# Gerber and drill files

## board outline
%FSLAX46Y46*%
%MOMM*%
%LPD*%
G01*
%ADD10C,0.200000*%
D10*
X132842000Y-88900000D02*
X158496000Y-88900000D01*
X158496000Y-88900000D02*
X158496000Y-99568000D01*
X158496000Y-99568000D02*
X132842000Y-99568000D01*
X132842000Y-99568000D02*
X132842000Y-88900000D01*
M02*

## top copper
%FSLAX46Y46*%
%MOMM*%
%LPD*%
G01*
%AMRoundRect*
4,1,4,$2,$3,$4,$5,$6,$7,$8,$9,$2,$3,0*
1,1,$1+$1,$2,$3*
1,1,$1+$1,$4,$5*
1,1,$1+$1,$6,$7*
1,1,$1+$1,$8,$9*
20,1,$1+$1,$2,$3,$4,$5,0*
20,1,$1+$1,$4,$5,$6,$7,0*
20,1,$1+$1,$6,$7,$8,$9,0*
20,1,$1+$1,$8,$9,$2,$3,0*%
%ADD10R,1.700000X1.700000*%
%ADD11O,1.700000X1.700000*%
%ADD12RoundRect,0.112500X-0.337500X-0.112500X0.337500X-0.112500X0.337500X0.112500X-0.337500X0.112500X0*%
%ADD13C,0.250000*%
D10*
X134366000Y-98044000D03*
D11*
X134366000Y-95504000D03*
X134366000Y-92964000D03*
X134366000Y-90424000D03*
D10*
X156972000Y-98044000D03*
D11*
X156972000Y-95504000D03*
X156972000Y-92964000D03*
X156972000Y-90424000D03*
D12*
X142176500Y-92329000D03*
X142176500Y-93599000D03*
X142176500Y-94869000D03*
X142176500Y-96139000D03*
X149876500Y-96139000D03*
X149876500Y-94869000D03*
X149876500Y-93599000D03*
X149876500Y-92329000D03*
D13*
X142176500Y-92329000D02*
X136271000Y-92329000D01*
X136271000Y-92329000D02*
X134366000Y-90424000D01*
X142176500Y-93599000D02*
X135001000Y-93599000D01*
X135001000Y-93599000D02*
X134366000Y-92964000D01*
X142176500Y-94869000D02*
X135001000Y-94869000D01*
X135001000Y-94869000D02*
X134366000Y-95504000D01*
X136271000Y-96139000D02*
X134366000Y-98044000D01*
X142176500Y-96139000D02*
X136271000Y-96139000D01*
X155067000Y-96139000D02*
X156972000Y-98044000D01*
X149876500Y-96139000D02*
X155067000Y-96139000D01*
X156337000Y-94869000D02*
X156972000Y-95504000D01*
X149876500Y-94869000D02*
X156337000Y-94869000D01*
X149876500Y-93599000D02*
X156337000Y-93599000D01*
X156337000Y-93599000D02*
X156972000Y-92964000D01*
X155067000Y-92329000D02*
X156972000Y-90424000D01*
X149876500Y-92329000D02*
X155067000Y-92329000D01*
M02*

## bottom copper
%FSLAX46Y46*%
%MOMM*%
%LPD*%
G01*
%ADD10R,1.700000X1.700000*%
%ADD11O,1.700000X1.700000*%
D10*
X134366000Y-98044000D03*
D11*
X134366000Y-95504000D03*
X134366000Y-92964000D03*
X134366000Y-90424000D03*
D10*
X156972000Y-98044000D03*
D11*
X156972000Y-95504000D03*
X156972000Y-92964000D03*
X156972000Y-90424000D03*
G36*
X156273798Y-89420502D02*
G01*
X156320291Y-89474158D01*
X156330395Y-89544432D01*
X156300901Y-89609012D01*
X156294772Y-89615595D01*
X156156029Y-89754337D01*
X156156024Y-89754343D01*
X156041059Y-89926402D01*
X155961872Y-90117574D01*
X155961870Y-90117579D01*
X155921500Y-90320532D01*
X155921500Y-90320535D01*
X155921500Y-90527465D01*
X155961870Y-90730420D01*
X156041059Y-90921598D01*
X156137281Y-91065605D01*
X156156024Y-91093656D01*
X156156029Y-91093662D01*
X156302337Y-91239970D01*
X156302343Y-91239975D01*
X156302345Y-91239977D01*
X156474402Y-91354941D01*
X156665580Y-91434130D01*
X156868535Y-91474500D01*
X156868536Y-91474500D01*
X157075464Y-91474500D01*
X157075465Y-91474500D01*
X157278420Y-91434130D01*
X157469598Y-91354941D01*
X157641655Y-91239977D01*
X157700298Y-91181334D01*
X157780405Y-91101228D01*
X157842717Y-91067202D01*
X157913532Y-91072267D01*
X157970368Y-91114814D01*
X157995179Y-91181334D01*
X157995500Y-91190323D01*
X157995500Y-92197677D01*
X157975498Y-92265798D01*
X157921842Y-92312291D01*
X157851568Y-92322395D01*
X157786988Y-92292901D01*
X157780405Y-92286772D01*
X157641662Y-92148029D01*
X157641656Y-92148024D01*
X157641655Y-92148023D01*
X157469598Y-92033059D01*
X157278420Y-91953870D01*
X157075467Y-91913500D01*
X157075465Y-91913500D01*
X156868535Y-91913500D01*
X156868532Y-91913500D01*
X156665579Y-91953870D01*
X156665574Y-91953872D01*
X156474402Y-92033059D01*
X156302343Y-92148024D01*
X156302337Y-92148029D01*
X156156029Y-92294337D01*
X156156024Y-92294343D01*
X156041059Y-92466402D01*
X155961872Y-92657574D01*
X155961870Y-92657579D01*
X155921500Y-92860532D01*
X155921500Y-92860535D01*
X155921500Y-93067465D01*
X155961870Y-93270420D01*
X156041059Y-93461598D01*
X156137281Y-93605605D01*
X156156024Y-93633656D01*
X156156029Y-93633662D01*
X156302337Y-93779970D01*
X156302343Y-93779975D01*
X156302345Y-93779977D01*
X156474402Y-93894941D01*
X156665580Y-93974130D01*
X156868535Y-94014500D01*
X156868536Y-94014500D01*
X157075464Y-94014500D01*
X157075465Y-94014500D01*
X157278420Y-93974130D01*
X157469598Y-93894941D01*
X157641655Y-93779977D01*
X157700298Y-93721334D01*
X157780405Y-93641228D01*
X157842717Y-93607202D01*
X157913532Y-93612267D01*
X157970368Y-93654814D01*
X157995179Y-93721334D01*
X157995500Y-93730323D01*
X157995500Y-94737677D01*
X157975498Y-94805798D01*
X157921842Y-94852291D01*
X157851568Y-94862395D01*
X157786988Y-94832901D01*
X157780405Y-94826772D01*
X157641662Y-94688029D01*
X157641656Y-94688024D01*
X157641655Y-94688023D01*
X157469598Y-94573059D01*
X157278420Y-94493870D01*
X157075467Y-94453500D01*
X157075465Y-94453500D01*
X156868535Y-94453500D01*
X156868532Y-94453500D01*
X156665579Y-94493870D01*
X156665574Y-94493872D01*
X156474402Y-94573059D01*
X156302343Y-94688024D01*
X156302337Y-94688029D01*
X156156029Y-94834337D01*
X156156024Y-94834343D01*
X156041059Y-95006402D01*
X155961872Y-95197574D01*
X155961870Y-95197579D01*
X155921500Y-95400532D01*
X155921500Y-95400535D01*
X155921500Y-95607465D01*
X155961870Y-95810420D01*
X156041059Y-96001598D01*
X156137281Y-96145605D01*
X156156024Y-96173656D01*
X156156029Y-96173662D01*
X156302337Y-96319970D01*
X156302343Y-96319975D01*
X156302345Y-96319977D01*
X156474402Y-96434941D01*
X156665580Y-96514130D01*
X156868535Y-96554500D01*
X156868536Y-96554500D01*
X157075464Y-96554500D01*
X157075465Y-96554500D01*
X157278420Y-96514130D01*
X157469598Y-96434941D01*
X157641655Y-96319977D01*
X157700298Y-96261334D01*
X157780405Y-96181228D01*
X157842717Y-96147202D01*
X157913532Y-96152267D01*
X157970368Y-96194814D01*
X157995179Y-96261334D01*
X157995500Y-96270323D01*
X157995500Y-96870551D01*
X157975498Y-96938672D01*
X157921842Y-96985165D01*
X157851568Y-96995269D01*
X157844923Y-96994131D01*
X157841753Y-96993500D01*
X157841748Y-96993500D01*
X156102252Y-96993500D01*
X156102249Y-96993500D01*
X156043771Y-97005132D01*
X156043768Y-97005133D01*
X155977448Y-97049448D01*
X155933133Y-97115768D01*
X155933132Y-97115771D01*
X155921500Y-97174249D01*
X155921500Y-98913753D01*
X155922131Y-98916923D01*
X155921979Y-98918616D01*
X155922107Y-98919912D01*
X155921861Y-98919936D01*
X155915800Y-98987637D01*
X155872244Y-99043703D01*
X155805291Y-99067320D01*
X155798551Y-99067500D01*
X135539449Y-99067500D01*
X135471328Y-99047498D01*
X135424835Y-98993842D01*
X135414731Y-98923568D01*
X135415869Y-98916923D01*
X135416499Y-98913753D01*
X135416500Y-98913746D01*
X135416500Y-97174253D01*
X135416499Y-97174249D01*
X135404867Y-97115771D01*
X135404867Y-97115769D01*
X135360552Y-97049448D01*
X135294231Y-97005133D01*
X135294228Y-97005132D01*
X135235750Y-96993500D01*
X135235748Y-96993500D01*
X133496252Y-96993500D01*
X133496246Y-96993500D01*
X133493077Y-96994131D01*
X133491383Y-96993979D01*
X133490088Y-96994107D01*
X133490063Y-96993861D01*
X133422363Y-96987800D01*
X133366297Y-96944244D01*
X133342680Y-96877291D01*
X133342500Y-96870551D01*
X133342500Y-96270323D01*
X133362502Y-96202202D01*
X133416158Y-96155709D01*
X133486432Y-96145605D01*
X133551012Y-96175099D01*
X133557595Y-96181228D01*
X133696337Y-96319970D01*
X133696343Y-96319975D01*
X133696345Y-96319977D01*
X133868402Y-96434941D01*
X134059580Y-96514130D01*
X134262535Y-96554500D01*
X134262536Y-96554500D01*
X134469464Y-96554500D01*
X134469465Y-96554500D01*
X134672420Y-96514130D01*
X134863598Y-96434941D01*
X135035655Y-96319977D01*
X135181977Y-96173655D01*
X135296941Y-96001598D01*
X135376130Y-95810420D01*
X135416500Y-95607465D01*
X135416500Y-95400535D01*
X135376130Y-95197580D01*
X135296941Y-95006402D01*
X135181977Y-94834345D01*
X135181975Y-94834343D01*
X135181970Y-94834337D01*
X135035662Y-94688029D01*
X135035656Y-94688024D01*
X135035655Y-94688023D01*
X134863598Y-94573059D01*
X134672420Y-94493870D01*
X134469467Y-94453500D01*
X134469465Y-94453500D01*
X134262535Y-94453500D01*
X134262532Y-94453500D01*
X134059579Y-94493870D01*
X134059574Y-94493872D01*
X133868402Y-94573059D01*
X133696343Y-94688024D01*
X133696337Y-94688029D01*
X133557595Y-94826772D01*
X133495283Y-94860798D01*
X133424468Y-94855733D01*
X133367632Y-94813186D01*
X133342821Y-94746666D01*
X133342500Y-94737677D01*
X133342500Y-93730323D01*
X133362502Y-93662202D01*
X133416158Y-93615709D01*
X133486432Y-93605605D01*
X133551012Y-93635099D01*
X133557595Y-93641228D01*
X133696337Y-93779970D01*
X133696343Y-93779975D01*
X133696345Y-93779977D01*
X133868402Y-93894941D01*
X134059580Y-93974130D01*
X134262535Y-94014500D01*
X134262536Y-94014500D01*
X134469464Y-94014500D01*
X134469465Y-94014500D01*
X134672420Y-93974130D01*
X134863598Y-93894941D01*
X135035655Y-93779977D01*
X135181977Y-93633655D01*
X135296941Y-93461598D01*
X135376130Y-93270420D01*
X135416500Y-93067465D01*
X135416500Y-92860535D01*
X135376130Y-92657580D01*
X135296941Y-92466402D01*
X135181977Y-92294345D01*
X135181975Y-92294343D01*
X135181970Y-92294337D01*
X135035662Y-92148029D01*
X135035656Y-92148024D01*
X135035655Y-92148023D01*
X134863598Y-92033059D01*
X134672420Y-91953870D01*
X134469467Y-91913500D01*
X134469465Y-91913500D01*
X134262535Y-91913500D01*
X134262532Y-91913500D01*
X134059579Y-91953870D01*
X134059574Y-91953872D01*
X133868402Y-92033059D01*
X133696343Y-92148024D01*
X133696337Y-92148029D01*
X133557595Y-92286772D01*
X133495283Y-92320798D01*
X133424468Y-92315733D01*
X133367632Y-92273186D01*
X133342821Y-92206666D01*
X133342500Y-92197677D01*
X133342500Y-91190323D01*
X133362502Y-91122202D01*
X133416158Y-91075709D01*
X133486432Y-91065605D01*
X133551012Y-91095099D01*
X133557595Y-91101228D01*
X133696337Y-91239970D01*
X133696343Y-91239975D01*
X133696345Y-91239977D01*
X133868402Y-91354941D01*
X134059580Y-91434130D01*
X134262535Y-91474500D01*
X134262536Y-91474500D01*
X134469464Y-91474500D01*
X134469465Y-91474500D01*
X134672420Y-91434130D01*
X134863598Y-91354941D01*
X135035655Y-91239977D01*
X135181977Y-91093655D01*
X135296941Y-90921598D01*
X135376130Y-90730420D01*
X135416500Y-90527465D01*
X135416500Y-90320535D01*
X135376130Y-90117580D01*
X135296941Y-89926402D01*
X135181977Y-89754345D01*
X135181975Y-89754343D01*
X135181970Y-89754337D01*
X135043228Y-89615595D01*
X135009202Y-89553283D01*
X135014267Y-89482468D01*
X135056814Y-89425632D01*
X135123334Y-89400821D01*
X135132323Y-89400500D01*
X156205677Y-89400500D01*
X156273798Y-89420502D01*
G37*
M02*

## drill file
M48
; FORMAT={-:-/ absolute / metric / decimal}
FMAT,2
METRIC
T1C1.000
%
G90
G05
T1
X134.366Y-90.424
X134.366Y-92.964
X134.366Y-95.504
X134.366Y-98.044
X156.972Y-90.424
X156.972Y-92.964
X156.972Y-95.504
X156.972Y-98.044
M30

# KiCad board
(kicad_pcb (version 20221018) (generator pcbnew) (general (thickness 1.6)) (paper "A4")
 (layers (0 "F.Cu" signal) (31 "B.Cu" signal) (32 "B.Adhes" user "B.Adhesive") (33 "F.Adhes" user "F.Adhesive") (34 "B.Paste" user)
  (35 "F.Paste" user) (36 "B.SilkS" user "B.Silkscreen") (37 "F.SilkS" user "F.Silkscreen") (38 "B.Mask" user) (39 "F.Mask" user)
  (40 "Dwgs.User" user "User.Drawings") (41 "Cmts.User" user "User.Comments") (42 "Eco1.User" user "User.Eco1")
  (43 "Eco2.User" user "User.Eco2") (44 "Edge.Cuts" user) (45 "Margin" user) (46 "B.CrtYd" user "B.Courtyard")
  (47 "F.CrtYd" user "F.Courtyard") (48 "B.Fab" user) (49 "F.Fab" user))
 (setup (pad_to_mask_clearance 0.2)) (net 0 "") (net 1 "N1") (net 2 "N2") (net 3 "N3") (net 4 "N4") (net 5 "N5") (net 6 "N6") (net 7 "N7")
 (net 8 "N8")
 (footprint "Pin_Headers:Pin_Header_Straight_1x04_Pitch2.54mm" (layer "F.Cu") (at 134.366 98.044 180)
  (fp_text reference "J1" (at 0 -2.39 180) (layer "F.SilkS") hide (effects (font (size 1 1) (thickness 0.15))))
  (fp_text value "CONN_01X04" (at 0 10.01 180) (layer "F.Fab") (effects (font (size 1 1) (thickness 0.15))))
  (pad "1" thru_hole rect (at 0 0 180) (size 1.7 1.7) (drill 1) (layers "*.Cu" "*.Mask") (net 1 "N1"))
  (pad "2" thru_hole oval (at 0 2.54 180) (size 1.7 1.7) (drill 1) (layers "*.Cu" "*.Mask") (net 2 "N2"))
  (pad "3" thru_hole oval (at 0 5.08 180) (size 1.7 1.7) (drill 1) (layers "*.Cu" "*.Mask") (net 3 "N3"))
  (pad "4" thru_hole oval (at 0 7.62 180) (size 1.7 1.7) (drill 1) (layers "*.Cu" "*.Mask") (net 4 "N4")))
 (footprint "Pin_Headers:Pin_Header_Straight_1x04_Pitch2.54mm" (layer "F.Cu") (at 156.972 98.044 180)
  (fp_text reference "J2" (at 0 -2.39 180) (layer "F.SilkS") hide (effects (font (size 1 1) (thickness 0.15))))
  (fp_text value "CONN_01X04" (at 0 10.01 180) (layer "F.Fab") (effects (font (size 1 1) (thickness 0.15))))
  (pad "1" thru_hole rect (at 0 0 180) (size 1.7 1.7) (drill 1) (layers "*.Cu" "*.Mask") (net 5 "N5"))
  (pad "2" thru_hole oval (at 0 2.54 180) (size 1.7 1.7) (drill 1) (layers "*.Cu" "*.Mask") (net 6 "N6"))
  (pad "3" thru_hole oval (at 0 5.08 180) (size 1.7 1.7) (drill 1) (layers "*.Cu" "*.Mask") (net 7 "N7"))
  (pad "4" thru_hole oval (at 0 7.62 180) (size 1.7 1.7) (drill 1) (layers "*.Cu" "*.Mask") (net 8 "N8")))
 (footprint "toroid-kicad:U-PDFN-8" (layer "F.Cu") (at 146.05 94.234)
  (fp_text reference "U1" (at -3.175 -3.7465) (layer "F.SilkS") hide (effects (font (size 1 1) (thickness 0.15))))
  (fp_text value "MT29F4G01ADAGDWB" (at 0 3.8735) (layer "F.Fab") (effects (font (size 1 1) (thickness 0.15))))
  (pad "1" smd roundrect (at -3.8735 -1.905) (size 0.9 0.45) (layers "F.Cu" "F.Paste" "F.Mask") (roundrect_rratio 0.25) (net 4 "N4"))
  (pad "2" smd roundrect (at -3.8735 -0.635) (size 0.9 0.45) (layers "F.Cu" "F.Paste" "F.Mask") (roundrect_rratio 0.25) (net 3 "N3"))
  (pad "3" smd roundrect (at -3.8735 0.635) (size 0.9 0.45) (layers "F.Cu" "F.Paste" "F.Mask") (roundrect_rratio 0.25) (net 2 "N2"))
  (pad "4" smd roundrect (at -3.8735 1.905) (size 0.9 0.45) (layers "F.Cu" "F.Paste" "F.Mask") (roundrect_rratio 0.25) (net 1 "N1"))
  (pad "5" smd roundrect (at 3.8265 1.905) (size 0.9 0.45) (layers "F.Cu" "F.Paste" "F.Mask") (roundrect_rratio 0.25) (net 5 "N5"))
  (pad "6" smd roundrect (at 3.8265 0.635) (size 0.9 0.45) (layers "F.Cu" "F.Paste" "F.Mask") (roundrect_rratio 0.25) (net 6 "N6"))
  (pad "7" smd roundrect (at 3.8265 -0.635) (size 0.9 0.45) (layers "F.Cu" "F.Paste" "F.Mask") (roundrect_rratio 0.25) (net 7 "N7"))
  (pad "8" smd roundrect (at 3.8265 -1.905) (size 0.9 0.45) (layers "F.Cu" "F.Paste" "F.Mask") (roundrect_rratio 0.25) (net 8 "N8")))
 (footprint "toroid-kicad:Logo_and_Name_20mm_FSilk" (layer "B.Cu") (at 145.542 94.234)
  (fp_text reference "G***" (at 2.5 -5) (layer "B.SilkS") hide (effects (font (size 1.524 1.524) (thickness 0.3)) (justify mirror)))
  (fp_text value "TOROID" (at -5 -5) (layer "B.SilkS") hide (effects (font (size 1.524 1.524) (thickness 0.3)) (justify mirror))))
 (gr_line (start 132.842 88.9) (end 158.496 88.9) (stroke (width 0.2) (type solid)) (layer "Edge.Cuts"))
 (gr_line (start 158.496 88.9) (end 158.496 99.568) (stroke (width 0.2) (type solid)) (layer "Edge.Cuts"))
 (gr_line (start 158.496 99.568) (end 132.842 99.568) (stroke (width 0.2) (type solid)) (layer "Edge.Cuts"))
 (gr_line (start 132.842 99.568) (end 132.842 88.9) (stroke (width 0.2) (type solid)) (layer "Edge.Cuts"))
 (segment (start 142.1765 92.329) (end 136.271 92.329) (width 0.25) (layer "F.Cu") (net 4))
 (segment (start 136.271 92.329) (end 134.366 90.424) (width 0.25) (layer "F.Cu") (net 4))
 (segment (start 142.1765 93.599) (end 135.001 93.599) (width 0.25) (layer "F.Cu") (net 3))
 (segment (start 135.001 93.599) (end 134.366 92.964) (width 0.25) (layer "F.Cu") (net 3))
 (segment (start 142.1765 94.869) (end 135.001 94.869) (width 0.25) (layer "F.Cu") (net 2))
 (segment (start 135.001 94.869) (end 134.366 95.504) (width 0.25) (layer "F.Cu") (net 2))
 (segment (start 136.271 96.139) (end 134.366 98.044) (width 0.25) (layer "F.Cu") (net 1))
 (segment (start 142.1765 96.139) (end 136.271 96.139) (width 0.25) (layer "F.Cu") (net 1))
 (segment (start 155.067 96.139) (end 156.972 98.044) (width 0.25) (layer "F.Cu") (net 5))
 (segment (start 149.8765 96.139) (end 155.067 96.139) (width 0.25) (layer "F.Cu") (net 5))
 (segment (start 156.337 94.869) (end 156.972 95.504) (width 0.25) (layer "F.Cu") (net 6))
 (segment (start 149.8765 94.869) (end 156.337 94.869) (width 0.25) (layer "F.Cu") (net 6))
 (segment (start 149.8765 93.599) (end 156.337 93.599) (width 0.25) (layer "F.Cu") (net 7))
 (segment (start 156.337 93.599) (end 156.972 92.964) (width 0.25) (layer "F.Cu") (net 7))
 (segment (start 155.067 92.329) (end 156.972 90.424) (width 0.25) (layer "F.Cu") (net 8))
 (segment (start 149.8765 92.329) (end 155.067 92.329) (width 0.25) (layer "F.Cu") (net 8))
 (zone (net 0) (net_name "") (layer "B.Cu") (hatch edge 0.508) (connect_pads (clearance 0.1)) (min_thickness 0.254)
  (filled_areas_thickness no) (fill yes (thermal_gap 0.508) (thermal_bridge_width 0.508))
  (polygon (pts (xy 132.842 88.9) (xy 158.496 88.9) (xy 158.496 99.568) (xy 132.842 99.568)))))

